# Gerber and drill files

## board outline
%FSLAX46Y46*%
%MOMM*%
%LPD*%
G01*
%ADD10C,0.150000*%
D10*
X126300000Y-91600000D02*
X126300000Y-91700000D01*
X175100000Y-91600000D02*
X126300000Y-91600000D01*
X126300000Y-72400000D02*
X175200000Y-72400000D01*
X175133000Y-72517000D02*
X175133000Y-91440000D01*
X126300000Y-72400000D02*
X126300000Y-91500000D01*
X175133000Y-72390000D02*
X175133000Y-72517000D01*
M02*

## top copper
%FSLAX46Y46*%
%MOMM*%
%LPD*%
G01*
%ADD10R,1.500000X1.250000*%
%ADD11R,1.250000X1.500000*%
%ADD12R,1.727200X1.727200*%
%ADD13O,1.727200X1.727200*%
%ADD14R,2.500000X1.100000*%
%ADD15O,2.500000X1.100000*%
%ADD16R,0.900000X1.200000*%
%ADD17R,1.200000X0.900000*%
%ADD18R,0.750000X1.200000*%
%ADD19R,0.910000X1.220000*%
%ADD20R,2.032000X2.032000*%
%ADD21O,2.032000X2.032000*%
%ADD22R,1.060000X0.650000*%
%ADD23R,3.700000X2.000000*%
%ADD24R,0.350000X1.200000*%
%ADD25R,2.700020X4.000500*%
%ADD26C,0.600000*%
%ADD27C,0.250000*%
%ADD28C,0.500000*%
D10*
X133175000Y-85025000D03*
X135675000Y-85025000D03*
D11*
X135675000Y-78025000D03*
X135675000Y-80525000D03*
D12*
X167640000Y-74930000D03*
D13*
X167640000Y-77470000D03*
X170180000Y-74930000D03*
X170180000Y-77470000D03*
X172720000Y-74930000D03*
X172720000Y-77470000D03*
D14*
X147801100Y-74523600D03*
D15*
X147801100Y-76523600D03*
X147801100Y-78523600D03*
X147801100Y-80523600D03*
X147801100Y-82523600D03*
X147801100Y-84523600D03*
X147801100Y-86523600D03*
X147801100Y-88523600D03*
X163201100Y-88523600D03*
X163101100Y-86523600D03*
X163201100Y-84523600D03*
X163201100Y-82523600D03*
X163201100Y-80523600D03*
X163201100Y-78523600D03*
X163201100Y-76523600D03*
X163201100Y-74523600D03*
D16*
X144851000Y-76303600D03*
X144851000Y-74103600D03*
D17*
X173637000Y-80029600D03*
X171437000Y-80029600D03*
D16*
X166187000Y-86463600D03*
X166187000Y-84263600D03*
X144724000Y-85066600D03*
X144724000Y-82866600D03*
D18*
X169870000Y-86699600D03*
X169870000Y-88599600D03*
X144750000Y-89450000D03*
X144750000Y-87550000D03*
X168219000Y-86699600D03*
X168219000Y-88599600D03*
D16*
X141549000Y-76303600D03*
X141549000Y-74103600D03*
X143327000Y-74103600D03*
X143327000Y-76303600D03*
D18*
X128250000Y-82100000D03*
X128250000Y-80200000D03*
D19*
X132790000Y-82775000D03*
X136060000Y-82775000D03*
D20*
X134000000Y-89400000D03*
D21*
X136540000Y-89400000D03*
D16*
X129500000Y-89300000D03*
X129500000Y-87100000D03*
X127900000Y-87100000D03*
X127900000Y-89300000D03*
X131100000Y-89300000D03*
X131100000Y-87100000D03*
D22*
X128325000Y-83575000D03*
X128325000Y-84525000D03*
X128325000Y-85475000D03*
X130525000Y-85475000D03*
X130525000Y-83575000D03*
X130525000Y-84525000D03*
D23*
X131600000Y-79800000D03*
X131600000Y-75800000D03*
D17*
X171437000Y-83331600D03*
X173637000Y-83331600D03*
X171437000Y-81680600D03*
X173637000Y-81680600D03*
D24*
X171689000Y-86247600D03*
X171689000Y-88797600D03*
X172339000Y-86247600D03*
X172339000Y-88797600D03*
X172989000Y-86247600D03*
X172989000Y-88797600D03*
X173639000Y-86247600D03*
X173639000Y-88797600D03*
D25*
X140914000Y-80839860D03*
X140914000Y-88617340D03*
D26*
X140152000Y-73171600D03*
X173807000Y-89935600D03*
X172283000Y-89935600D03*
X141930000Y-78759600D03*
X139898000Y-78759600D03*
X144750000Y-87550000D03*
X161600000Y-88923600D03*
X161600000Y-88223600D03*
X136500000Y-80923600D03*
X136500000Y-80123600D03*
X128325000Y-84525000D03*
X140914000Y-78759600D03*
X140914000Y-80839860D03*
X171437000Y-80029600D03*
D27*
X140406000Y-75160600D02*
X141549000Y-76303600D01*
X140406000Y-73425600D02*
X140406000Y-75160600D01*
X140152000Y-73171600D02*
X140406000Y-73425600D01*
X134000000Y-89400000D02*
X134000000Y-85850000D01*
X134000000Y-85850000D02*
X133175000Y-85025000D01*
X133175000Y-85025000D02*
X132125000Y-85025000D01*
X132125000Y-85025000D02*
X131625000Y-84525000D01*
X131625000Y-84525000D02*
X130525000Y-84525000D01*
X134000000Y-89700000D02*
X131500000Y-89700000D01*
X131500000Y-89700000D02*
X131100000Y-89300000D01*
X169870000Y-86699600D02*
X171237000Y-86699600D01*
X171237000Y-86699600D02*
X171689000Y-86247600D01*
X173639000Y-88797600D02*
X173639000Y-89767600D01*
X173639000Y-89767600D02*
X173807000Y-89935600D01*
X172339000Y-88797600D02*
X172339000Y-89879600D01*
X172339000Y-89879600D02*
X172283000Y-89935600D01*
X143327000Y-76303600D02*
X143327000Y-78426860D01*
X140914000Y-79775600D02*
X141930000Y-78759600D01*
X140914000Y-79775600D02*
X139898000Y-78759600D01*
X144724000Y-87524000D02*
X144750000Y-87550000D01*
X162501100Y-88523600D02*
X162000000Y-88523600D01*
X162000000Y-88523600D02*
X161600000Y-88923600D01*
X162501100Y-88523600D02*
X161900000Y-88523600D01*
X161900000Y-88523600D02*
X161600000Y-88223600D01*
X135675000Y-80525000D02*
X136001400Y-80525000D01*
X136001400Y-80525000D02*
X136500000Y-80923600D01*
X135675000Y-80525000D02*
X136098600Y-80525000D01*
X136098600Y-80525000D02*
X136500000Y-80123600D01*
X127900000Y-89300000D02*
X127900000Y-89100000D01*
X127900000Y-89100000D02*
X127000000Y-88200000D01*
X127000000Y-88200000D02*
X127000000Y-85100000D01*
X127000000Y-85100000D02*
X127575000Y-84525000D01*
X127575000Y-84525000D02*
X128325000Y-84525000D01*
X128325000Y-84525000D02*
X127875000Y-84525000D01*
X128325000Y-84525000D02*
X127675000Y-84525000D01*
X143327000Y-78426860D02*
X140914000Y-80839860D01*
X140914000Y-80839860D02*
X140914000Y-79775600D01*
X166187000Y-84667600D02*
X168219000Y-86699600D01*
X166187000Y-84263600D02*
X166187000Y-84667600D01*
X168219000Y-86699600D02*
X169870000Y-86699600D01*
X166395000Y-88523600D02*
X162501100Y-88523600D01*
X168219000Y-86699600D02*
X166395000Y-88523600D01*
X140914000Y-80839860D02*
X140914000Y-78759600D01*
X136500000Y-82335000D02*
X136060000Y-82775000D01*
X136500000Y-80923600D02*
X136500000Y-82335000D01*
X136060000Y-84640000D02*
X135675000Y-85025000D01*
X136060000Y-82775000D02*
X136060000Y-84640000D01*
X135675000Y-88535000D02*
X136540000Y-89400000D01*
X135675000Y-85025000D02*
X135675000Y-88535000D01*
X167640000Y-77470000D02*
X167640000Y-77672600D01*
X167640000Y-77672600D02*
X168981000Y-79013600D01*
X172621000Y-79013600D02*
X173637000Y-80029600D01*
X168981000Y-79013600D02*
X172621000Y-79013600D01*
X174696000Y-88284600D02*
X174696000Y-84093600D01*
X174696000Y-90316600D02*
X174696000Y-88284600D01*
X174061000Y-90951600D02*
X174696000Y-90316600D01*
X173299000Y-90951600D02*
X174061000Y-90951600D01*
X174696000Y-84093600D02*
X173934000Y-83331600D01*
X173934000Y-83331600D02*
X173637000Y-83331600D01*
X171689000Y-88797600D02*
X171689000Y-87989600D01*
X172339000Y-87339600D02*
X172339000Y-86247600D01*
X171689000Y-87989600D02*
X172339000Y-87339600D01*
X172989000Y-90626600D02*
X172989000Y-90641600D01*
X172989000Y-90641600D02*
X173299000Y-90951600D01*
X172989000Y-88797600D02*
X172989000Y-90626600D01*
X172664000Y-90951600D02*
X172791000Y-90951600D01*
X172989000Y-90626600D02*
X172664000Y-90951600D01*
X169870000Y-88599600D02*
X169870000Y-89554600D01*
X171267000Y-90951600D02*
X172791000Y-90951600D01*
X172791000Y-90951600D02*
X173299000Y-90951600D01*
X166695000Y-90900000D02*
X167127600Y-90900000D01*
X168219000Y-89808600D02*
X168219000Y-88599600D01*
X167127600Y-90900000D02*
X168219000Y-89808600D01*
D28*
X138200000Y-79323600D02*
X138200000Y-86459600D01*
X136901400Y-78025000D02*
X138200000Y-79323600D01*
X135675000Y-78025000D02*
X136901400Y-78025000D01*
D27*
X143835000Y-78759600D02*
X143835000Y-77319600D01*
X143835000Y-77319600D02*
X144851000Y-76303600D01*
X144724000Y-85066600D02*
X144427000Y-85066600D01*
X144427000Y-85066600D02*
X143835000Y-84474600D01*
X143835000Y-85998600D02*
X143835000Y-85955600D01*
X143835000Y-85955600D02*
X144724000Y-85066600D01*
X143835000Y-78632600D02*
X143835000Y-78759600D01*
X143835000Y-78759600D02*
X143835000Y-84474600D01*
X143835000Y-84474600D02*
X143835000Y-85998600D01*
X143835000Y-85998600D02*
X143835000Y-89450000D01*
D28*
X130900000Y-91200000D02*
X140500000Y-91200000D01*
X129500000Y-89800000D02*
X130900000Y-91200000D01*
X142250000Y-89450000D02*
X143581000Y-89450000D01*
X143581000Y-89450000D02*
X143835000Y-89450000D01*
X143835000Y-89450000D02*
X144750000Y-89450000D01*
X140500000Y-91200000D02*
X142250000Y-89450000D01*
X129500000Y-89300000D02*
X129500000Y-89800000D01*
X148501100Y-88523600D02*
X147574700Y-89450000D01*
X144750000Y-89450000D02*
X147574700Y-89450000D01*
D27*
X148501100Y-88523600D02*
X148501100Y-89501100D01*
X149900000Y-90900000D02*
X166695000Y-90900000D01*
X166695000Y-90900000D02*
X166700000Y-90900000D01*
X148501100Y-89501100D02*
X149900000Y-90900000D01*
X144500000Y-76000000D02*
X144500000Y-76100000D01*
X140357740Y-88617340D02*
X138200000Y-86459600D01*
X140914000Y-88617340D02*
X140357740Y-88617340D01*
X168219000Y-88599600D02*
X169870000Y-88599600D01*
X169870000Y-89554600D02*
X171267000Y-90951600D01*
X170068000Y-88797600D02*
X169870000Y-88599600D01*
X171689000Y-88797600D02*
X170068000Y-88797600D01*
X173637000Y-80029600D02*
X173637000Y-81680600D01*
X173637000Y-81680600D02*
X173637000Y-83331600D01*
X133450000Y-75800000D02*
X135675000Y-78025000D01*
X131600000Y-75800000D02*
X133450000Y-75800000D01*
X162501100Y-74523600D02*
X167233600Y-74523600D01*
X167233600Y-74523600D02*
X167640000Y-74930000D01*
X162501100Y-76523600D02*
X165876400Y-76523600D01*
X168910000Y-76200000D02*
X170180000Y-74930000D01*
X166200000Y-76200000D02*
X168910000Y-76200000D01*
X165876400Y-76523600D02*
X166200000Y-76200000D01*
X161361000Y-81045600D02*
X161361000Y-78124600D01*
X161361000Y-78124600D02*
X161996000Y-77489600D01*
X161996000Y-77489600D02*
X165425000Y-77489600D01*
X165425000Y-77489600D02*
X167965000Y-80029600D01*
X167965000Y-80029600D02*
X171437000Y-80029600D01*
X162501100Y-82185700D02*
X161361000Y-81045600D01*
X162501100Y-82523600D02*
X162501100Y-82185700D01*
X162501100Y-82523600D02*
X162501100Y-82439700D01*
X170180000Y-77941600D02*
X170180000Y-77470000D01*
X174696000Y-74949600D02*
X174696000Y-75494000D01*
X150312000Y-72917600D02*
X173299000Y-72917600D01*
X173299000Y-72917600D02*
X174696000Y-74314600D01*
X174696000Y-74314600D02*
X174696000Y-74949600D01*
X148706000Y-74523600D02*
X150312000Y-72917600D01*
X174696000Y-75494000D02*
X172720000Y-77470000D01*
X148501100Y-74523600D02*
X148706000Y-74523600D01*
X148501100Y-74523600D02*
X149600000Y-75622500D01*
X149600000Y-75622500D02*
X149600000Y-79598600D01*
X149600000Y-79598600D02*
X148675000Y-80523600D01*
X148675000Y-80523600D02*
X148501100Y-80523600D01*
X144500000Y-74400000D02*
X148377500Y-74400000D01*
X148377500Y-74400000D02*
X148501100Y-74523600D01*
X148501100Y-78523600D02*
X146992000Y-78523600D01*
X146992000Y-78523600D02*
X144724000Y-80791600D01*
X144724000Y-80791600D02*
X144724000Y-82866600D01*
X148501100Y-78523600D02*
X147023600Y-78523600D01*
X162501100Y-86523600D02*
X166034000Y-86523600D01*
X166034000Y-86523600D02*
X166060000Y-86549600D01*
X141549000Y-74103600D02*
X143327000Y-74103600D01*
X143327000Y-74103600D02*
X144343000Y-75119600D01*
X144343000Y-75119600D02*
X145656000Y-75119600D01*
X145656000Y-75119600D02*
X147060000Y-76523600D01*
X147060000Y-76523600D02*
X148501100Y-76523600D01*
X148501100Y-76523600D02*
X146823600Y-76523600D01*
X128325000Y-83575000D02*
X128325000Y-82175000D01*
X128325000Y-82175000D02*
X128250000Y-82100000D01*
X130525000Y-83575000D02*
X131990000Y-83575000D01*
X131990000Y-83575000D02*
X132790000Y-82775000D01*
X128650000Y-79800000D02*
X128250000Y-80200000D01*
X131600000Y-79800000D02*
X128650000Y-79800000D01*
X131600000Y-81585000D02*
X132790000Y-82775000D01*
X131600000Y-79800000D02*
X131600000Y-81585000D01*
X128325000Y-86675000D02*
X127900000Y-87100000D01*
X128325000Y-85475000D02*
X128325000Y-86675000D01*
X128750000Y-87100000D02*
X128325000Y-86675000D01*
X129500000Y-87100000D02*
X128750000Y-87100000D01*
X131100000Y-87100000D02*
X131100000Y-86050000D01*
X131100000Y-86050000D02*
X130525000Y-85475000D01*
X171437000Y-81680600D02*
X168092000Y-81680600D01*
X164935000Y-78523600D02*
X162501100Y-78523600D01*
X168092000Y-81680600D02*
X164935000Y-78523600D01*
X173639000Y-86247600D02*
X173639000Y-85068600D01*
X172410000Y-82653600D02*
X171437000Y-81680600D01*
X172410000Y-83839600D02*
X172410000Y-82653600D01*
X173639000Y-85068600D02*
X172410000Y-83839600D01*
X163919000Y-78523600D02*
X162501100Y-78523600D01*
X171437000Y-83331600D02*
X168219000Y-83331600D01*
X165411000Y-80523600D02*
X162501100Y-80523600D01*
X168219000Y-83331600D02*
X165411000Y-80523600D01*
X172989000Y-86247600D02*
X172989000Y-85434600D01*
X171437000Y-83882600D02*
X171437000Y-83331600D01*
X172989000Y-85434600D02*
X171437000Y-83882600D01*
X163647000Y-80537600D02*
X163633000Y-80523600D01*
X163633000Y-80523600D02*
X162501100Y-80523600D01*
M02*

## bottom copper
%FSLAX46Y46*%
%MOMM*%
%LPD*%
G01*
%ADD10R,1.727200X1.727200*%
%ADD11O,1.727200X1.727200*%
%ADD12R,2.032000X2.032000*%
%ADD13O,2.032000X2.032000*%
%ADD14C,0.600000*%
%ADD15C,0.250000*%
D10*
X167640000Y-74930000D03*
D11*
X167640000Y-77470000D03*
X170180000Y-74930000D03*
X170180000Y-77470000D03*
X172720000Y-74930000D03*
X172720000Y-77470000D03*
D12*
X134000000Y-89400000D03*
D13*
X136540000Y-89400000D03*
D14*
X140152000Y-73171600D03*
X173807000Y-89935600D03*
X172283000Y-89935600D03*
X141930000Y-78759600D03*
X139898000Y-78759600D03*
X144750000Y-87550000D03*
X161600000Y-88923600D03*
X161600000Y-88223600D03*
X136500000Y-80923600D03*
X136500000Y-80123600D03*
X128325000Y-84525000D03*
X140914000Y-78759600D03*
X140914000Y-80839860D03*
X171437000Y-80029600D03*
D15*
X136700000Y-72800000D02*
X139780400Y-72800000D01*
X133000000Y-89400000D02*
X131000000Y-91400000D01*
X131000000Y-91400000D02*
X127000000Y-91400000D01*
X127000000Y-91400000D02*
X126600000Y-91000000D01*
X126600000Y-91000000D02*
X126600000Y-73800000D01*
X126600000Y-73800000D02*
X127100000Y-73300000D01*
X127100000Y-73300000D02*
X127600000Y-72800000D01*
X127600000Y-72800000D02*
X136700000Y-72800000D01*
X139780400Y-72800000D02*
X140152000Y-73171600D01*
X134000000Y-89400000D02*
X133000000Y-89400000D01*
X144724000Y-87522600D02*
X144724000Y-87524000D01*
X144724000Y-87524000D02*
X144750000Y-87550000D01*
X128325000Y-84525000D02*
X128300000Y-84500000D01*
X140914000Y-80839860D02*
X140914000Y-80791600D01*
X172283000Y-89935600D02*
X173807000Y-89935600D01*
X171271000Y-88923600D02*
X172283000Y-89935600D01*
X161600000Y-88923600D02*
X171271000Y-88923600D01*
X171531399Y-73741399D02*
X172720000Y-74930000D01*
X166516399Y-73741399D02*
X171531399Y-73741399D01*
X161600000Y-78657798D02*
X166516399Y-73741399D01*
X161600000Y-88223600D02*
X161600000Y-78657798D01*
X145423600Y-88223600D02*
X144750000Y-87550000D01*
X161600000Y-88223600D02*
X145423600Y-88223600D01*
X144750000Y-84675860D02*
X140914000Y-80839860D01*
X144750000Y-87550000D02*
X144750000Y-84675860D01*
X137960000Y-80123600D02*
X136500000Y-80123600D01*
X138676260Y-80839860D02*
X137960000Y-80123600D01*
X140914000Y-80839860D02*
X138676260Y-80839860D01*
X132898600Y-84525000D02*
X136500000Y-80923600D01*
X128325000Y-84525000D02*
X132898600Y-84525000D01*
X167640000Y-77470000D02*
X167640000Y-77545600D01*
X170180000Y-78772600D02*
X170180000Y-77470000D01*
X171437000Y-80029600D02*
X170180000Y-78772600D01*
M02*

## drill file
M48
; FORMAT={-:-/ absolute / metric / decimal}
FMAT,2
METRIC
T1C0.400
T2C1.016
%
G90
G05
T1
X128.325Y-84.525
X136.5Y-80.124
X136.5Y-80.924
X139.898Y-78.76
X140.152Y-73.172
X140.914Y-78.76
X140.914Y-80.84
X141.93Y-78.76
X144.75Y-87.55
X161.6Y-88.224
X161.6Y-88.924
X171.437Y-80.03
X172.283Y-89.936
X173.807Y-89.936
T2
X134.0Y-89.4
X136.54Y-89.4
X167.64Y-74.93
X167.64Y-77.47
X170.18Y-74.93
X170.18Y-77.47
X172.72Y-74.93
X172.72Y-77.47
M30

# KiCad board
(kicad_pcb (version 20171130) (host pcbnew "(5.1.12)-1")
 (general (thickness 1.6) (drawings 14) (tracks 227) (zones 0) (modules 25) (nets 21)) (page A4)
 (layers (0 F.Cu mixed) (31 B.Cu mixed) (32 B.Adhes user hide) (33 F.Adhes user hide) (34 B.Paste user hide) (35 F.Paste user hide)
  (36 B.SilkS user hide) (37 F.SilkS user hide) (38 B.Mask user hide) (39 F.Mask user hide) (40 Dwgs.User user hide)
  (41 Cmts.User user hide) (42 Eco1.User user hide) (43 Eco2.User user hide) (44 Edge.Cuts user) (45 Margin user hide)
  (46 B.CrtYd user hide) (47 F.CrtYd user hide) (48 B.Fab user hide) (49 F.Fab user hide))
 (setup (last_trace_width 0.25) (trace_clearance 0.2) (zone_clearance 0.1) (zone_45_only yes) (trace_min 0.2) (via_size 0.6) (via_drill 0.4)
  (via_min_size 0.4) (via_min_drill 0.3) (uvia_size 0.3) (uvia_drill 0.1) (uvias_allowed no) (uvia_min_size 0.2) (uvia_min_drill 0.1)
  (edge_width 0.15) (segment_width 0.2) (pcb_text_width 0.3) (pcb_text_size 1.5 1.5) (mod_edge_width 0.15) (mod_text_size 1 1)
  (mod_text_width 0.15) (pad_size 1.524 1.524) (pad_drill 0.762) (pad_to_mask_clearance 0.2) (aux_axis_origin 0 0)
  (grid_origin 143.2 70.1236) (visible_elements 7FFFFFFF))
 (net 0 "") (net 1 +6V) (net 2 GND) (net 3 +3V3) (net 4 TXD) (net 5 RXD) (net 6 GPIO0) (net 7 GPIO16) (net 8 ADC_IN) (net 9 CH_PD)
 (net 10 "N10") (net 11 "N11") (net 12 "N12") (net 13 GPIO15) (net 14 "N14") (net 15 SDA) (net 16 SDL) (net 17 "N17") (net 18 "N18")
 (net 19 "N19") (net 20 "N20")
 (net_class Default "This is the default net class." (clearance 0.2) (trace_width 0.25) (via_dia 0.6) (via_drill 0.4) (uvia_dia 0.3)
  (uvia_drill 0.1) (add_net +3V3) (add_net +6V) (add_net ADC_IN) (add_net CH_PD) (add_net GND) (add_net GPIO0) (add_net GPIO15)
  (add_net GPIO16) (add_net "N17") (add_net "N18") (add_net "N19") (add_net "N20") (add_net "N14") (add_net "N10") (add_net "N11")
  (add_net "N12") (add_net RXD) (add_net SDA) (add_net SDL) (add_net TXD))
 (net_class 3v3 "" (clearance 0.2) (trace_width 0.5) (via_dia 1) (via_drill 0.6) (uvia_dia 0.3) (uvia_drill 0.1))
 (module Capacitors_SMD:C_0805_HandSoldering (layer F.Cu) (at 134.425 85.025)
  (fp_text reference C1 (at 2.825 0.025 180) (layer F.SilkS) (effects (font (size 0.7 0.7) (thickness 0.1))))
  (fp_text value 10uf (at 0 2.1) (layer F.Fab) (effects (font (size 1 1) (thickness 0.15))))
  (pad 1 smd rect (at -1.25 0) (size 1.5 1.25) (layers F.Cu F.Paste F.Mask) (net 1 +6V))
  (pad 2 smd rect (at 1.25 0) (size 1.5 1.25) (layers F.Cu F.Paste F.Mask) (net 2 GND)))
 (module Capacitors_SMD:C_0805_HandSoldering (layer F.Cu) (at 135.675 79.275 270)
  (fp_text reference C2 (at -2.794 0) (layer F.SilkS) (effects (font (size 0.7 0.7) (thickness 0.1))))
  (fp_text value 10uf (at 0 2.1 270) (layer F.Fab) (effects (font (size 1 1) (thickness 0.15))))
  (pad 1 smd rect (at -1.25 0 270) (size 1.5 1.25) (layers F.Cu F.Paste F.Mask) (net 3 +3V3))
  (pad 2 smd rect (at 1.25 0 270) (size 1.5 1.25) (layers F.Cu F.Paste F.Mask) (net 2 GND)))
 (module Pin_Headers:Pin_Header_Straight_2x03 (layer B.Cu) (at 167.64 74.93 270)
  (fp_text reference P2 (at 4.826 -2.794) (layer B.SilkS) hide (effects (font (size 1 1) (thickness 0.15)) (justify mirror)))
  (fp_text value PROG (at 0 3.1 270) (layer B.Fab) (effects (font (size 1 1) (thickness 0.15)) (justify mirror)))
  (pad 1 thru_hole rect (at 0 0 270) (size 1.7272 1.7272) (drill 1.016) (layers *.Cu *.Mask B.SilkS) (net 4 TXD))
  (pad 2 thru_hole oval (at 2.54 0 270) (size 1.7272 1.7272) (drill 1.016) (layers *.Cu *.Mask B.SilkS) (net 3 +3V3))
  (pad 3 thru_hole oval (at 0 -2.54 270) (size 1.7272 1.7272) (drill 1.016) (layers *.Cu *.Mask B.SilkS) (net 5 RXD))
  (pad 4 thru_hole oval (at 2.54 -2.54 270) (size 1.7272 1.7272) (drill 1.016) (layers *.Cu *.Mask B.SilkS) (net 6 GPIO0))
  (pad 5 thru_hole oval (at 0 -5.08 270) (size 1.7272 1.7272) (drill 1.016) (layers *.Cu *.Mask B.SilkS) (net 2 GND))
  (pad 6 thru_hole oval (at 2.54 -5.08 270) (size 1.7272 1.7272) (drill 1.016) (layers *.Cu *.Mask B.SilkS) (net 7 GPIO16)))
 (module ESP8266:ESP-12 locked (layer F.Cu) (at 148.5011 74.5236)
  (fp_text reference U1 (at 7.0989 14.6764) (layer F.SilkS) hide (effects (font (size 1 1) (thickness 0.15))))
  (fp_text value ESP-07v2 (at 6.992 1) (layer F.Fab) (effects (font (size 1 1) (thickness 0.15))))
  (pad 1 smd rect (at 0 0) (size 2.5 1.1) (drill (offset -0.7 0)) (layers F.Cu F.Paste F.Mask) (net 7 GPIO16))
  (pad 2 smd oval (at 0 2) (size 2.5 1.1) (drill (offset -0.7 0)) (layers F.Cu F.Paste F.Mask) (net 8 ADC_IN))
  (pad 3 smd oval (at 0 4) (size 2.5 1.1) (drill (offset -0.7 0)) (layers F.Cu F.Paste F.Mask) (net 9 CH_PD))
  (pad 4 smd oval (at 0 6) (size 2.5 1.1) (drill (offset -0.7 0)) (layers F.Cu F.Paste F.Mask) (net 7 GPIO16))
  (pad 5 smd oval (at 0 8) (size 2.5 1.1) (drill (offset -0.7 0)) (layers F.Cu F.Paste F.Mask) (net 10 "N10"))
  (pad 6 smd oval (at 0 10) (size 2.5 1.1) (drill (offset -0.7 0)) (layers F.Cu F.Paste F.Mask) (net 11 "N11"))
  (pad 7 smd oval (at 0 12) (size 2.5 1.1) (drill (offset -0.7 0)) (layers F.Cu F.Paste F.Mask) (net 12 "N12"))
  (pad 8 smd oval (at 0 14) (size 2.5 1.1) (drill (offset -0.7 0)) (layers F.Cu F.Paste F.Mask) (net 3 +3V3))
  (pad 9 smd oval (at 14 14) (size 2.5 1.1) (drill (offset 0.7 0)) (layers F.Cu F.Paste F.Mask) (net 2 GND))
  (pad 10 smd oval (at 14 12) (size 2.5 1.1) (drill (offset 0.6 0)) (layers F.Cu F.Paste F.Mask) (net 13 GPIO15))
  (pad 11 smd oval (at 14 10) (size 2.5 1.1) (drill (offset 0.7 0)) (layers F.Cu F.Paste F.Mask) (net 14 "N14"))
  (pad 12 smd oval (at 14 8) (size 2.5 1.1) (drill (offset 0.7 0)) (layers F.Cu F.Paste F.Mask) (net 6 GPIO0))
  (pad 13 smd oval (at 14 6) (size 2.5 1.1) (drill (offset 0.7 0)) (layers F.Cu F.Paste F.Mask) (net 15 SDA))
  (pad 14 smd oval (at 14 4) (size 2.5 1.1) (drill (offset 0.7 0)) (layers F.Cu F.Paste F.Mask) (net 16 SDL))
  (pad 15 smd oval (at 14 2) (size 2.5 1.1) (drill (offset 0.7 0)) (layers F.Cu F.Paste F.Mask) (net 5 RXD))
  (pad 16 smd oval (at 14 0) (size 2.5 1.1) (drill (offset 0.7 0)) (layers F.Cu F.Paste F.Mask) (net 4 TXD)))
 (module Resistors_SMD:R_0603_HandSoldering (layer F.Cu) (at 144.851 75.2036 90)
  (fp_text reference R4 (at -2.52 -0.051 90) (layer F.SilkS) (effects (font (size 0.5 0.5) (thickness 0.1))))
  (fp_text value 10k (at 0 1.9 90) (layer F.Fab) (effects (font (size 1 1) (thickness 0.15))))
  (pad 1 smd rect (at -1.1 0 90) (size 1.2 0.9) (layers F.Cu F.Paste F.Mask) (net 3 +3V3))
  (pad 2 smd rect (at 1.1 0 90) (size 1.2 0.9) (layers F.Cu F.Paste F.Mask) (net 7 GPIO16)))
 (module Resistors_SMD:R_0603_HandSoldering (layer F.Cu) (at 172.537 80.0296 180)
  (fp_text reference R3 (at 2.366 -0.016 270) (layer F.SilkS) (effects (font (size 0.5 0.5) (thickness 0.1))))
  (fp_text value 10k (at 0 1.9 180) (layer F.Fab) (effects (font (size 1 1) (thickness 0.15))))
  (pad 1 smd rect (at -1.1 0 180) (size 1.2 0.9) (layers F.Cu F.Paste F.Mask) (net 3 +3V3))
  (pad 2 smd rect (at 1.1 0 180) (size 1.2 0.9) (layers F.Cu F.Paste F.Mask) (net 6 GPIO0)))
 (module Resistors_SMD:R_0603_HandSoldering (layer F.Cu) (at 166.187 85.3636 90)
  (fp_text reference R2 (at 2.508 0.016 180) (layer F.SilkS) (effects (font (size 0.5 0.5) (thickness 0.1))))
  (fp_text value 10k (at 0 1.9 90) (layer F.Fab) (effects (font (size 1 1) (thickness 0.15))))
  (pad 1 smd rect (at -1.1 0 90) (size 1.2 0.9) (layers F.Cu F.Paste F.Mask) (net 13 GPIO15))
  (pad 2 smd rect (at 1.1 0 90) (size 1.2 0.9) (layers F.Cu F.Paste F.Mask) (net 2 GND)))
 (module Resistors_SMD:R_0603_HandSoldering (layer F.Cu) (at 144.724 83.9666 90)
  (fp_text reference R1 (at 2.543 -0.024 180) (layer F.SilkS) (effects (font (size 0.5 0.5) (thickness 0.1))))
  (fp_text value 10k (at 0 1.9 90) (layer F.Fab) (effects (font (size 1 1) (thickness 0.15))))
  (pad 1 smd rect (at -1.1 0 90) (size 1.2 0.9) (layers F.Cu F.Paste F.Mask) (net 3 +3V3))
  (pad 2 smd rect (at 1.1 0 90) (size 1.2 0.9) (layers F.Cu F.Paste F.Mask) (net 9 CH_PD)))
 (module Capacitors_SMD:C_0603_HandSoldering (layer F.Cu) (at 169.87 87.6496 270)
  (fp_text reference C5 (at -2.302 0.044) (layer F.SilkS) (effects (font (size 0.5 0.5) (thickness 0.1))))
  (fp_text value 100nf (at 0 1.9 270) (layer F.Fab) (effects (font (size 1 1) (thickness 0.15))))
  (pad 1 smd rect (at -0.95 0 270) (size 1.2 0.75) (layers F.Cu F.Paste F.Mask) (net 2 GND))
  (pad 2 smd rect (at 0.95 0 270) (size 1.2 0.75) (layers F.Cu F.Paste F.Mask) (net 3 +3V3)))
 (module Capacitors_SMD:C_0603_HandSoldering (layer F.Cu) (at 144.75 88.5 90)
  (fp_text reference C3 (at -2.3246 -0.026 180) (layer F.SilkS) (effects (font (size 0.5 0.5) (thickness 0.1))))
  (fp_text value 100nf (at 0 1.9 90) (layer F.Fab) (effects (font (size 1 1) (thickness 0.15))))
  (pad 1 smd rect (at -0.95 0 90) (size 1.2 0.75) (layers F.Cu F.Paste F.Mask) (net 3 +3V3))
  (pad 2 smd rect (at 0.95 0 90) (size 1.2 0.75) (layers F.Cu F.Paste F.Mask) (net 2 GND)))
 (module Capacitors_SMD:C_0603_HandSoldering (layer F.Cu) (at 168.219 87.6496 270)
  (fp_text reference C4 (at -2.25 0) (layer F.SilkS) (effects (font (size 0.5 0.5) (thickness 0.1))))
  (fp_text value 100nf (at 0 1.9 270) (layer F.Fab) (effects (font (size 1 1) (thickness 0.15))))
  (pad 1 smd rect (at -0.95 0 270) (size 1.2 0.75) (layers F.Cu F.Paste F.Mask) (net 2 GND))
  (pad 2 smd rect (at 0.95 0 270) (size 1.2 0.75) (layers F.Cu F.Paste F.Mask) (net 3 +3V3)))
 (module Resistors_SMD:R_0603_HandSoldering (layer F.Cu) (at 141.549 75.2036 90)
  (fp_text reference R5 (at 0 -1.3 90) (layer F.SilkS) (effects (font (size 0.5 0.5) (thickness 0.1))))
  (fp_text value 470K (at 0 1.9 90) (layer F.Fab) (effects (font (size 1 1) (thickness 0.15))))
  (pad 1 smd rect (at -1.1 0 90) (size 1.2 0.9) (layers F.Cu F.Paste F.Mask) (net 1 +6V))
  (pad 2 smd rect (at 1.1 0 90) (size 1.2 0.9) (layers F.Cu F.Paste F.Mask) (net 8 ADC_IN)))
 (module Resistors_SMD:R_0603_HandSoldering (layer F.Cu) (at 143.327 75.2036 270)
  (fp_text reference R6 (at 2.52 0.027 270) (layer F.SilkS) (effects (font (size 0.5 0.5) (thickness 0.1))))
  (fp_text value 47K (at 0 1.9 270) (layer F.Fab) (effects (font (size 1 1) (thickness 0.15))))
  (pad 1 smd rect (at -1.1 0 270) (size 1.2 0.9) (layers F.Cu F.Paste F.Mask) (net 8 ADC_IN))
  (pad 2 smd rect (at 1.1 0 270) (size 1.2 0.9) (layers F.Cu F.Paste F.Mask) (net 2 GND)))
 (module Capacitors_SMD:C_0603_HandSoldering (layer F.Cu) (at 128.25 81.15 90)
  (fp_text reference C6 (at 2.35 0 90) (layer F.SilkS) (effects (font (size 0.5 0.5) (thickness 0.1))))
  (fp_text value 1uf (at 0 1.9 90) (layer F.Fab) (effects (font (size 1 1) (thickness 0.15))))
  (pad 1 smd rect (at -0.95 0 90) (size 1.2 0.75) (layers F.Cu F.Paste F.Mask) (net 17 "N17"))
  (pad 2 smd rect (at 0.95 0 90) (size 1.2 0.75) (layers F.Cu F.Paste F.Mask) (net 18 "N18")))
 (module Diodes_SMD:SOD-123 (layer F.Cu) (at 134.425 82.775)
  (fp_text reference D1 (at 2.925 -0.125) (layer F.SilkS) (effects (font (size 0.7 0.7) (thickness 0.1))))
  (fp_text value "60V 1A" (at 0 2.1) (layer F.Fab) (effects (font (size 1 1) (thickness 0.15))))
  (pad 1 smd rect (at -1.635 0) (size 0.91 1.22) (layers F.Cu F.Paste F.Mask) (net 18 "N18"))
  (pad 2 smd rect (at 1.635 0) (size 0.91 1.22) (layers F.Cu F.Paste F.Mask) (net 2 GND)))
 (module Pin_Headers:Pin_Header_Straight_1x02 (layer F.Cu) (at 134 89.4 90)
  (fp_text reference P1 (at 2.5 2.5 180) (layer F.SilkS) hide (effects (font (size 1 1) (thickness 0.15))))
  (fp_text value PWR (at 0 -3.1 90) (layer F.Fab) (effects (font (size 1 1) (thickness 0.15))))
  (pad 1 thru_hole rect (at 0 0 90) (size 2.032 2.032) (drill 1.016) (layers *.Cu *.Mask F.SilkS) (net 1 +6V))
  (pad 2 thru_hole oval (at 0 2.54 90) (size 2.032 2.032) (drill 1.016) (layers *.Cu *.Mask F.SilkS) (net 2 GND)))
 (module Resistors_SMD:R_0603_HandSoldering (layer F.Cu) (at 129.5 88.2 90)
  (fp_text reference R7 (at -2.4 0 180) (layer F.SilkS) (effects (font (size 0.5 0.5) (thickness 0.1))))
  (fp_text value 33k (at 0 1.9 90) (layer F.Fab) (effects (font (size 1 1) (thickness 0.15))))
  (pad 1 smd rect (at -1.1 0 90) (size 1.2 0.9) (layers F.Cu F.Paste F.Mask) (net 3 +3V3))
  (pad 2 smd rect (at 1.1 0 90) (size 1.2 0.9) (layers F.Cu F.Paste F.Mask) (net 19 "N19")))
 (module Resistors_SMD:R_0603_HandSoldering (layer F.Cu) (at 127.9 88.2 270)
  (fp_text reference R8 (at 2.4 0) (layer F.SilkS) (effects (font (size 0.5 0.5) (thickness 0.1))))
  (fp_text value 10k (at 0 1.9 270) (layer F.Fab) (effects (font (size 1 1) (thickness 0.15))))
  (pad 1 smd rect (at -1.1 0 270) (size 1.2 0.9) (layers F.Cu F.Paste F.Mask) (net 19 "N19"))
  (pad 2 smd rect (at 1.1 0 270) (size 1.2 0.9) (layers F.Cu F.Paste F.Mask) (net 2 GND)))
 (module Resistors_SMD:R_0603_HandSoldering (layer F.Cu) (at 131.1 88.2 90)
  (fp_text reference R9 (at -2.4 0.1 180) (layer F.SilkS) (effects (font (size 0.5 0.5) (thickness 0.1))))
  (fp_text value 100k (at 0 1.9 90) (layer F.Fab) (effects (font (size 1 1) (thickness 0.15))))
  (pad 1 smd rect (at -1.1 0 90) (size 1.2 0.9) (layers F.Cu F.Paste F.Mask) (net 1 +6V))
  (pad 2 smd rect (at 1.1 0 90) (size 1.2 0.9) (layers F.Cu F.Paste F.Mask) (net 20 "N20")))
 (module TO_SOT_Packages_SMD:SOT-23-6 (layer F.Cu) (at 129.425 84.525) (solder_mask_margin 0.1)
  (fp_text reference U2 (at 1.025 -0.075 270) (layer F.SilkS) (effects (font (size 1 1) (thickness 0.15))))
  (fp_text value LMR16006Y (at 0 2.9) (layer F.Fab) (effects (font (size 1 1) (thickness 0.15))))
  (pad 1 smd rect (at -1.1 -0.95) (size 1.06 0.65) (layers F.Cu F.Paste F.Mask) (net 17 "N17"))
  (pad 2 smd rect (at -1.1 0) (size 1.06 0.65) (layers F.Cu F.Paste F.Mask) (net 2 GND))
  (pad 3 smd rect (at -1.1 0.95) (size 1.06 0.65) (layers F.Cu F.Paste F.Mask) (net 19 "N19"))
  (pad 4 smd rect (at 1.1 0.95) (size 1.06 0.65) (layers F.Cu F.Paste F.Mask) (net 20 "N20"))
  (pad 6 smd rect (at 1.1 -0.95) (size 1.06 0.65) (layers F.Cu F.Paste F.Mask) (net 18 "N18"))
  (pad 5 smd rect (at 1.1 0) (size 1.06 0.65) (layers F.Cu F.Paste F.Mask) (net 1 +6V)))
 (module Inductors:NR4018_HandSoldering (layer F.Cu) (at 131.6 77.8 90)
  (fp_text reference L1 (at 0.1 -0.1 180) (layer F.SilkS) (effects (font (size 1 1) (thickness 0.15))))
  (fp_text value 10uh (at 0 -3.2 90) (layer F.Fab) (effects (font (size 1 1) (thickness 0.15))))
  (pad 1 smd rect (at -2 0 90) (size 2 3.7) (layers F.Cu F.Paste F.Mask) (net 18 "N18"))
  (pad 2 smd rect (at 2 0 90) (size 2 3.7) (layers F.Cu F.Paste F.Mask) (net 3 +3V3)))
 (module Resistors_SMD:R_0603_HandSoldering (layer F.Cu) (at 172.537 83.3316)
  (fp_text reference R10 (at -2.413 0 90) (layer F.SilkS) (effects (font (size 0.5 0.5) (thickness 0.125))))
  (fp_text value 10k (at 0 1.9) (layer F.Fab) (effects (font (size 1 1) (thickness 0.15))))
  (pad 1 smd rect (at -1.1 0) (size 1.2 0.9) (layers F.Cu F.Paste F.Mask) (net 15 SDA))
  (pad 2 smd rect (at 1.1 0) (size 1.2 0.9) (layers F.Cu F.Paste F.Mask) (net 3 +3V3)))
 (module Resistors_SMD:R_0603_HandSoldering (layer F.Cu) (at 172.537 81.6806)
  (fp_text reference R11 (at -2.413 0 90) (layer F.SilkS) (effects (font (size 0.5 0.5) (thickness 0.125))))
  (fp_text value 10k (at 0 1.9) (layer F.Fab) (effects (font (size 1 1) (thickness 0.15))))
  (pad 1 smd rect (at -1.1 0) (size 1.2 0.9) (layers F.Cu F.Paste F.Mask) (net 16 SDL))
  (pad 2 smd rect (at 1.1 0) (size 1.2 0.9) (layers F.Cu F.Paste F.Mask) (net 3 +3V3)))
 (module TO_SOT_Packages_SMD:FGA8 (layer F.Cu) (at 172.664 87.5226)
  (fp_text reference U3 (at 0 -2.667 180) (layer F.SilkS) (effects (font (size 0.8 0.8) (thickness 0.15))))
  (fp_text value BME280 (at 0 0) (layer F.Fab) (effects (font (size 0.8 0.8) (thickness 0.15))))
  (pad 1 smd rect (at -0.975 -1.275) (size 0.35 1.2) (layers F.Cu F.Paste F.Mask) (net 2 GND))
  (pad 8 smd rect (at -0.975 1.275) (size 0.35 1.2) (layers F.Cu F.Paste F.Mask) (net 3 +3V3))
  (pad 2 smd rect (at -0.325 -1.275) (size 0.35 1.2) (layers F.Cu F.Paste F.Mask) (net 3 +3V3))
  (pad 7 smd rect (at -0.325 1.275) (size 0.35 1.2) (layers F.Cu F.Paste F.Mask) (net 2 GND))
  (pad 3 smd rect (at 0.325 -1.275) (size 0.35 1.2) (layers F.Cu F.Paste F.Mask) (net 15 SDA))
  (pad 6 smd rect (at 0.325 1.275) (size 0.35 1.2) (layers F.Cu F.Paste F.Mask) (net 3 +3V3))
  (pad 4 smd rect (at 0.975 -1.275) (size 0.35 1.2) (layers F.Cu F.Paste F.Mask) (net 16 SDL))
  (pad 5 smd rect (at 0.975 1.275) (size 0.35 1.2) (layers F.Cu F.Paste F.Mask) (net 2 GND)))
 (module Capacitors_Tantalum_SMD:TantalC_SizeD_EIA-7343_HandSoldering (layer F.Cu) (at 140.914 84.7286 90)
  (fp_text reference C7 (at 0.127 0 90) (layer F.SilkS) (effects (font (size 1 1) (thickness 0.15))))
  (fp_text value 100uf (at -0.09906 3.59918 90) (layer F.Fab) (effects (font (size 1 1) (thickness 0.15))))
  (pad 2 smd rect (at 3.88874 0 90) (size 4.0005 2.70002) (layers F.Cu F.Paste F.Mask) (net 2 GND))
  (pad 1 smd rect (at -3.88874 0 90) (size 4.0005 2.70002) (layers F.Cu F.Paste F.Mask) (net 3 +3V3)))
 (gr_line (start 126.3 91.6) (end 126.3 91.7) (angle 90) (layer Edge.Cuts) (width 0.15))
 (gr_line (start 175.1 91.6) (end 126.3 91.6) (angle 90) (layer Edge.Cuts) (width 0.15))
 (gr_line (start 126.3 72.4) (end 175.2 72.4) (angle 90) (layer Edge.Cuts) (width 0.15))
 (gr_line (start 175.133 72.517) (end 175.133 91.44) (angle 90) (layer Edge.Cuts) (width 0.15))
 (gr_line (start 126.3 72.4) (end 126.3 91.5) (angle 90) (layer Edge.Cuts) (width 0.15))
 (gr_line (start 175.133 72.39) (end 175.133 72.517) (angle 90) (layer Edge.Cuts) (width 0.15))
 (segment (start 136.7 72.8) (end 139.7804 72.8) (width 0.25) (layer B.Cu) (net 1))
 (segment (start 133 89.4) (end 131 91.4) (width 0.25) (layer B.Cu) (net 1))
 (segment (start 131 91.4) (end 127 91.4) (width 0.25) (layer B.Cu) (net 1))
 (segment (start 127 91.4) (end 126.6 91) (width 0.25) (layer B.Cu) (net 1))
 (segment (start 126.6 91) (end 126.6 73.8) (width 0.25) (layer B.Cu) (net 1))
 (segment (start 126.6 73.8) (end 127.1 73.3) (width 0.25) (layer B.Cu) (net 1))
 (segment (start 127.1 73.3) (end 127.6 72.8) (width 0.25) (layer B.Cu) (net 1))
 (segment (start 127.6 72.8) (end 136.7 72.8) (width 0.25) (layer B.Cu) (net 1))
 (segment (start 140.406 75.1606) (end 141.549 76.3036) (width 0.25) (layer F.Cu) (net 1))
 (segment (start 140.406 73.4256) (end 140.406 75.1606) (width 0.25) (layer F.Cu) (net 1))
 (segment (start 140.152 73.1716) (end 140.406 73.4256) (width 0.25) (layer F.Cu) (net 1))
 (segment (start 139.7804 72.8) (end 140.152 73.1716) (width 0.25) (layer B.Cu) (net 1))
 (segment (start 134 89.4) (end 134 85.85) (width 0.25) (layer F.Cu) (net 1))
 (segment (start 134 85.85) (end 133.175 85.025) (width 0.25) (layer F.Cu) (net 1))
 (segment (start 134 89.4) (end 133 89.4) (width 0.25) (layer B.Cu) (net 1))
 (segment (start 133.175 85.025) (end 132.125 85.025) (width 0.25) (layer F.Cu) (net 1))
 (segment (start 132.125 85.025) (end 131.625 84.525) (width 0.25) (layer F.Cu) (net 1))
 (segment (start 131.625 84.525) (end 130.525 84.525) (width 0.25) (layer F.Cu) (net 1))
 (segment (start 134 89.7) (end 131.5 89.7) (width 0.25) (layer F.Cu) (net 1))
 (segment (start 131.5 89.7) (end 131.1 89.3) (width 0.25) (layer F.Cu) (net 1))
 (segment (start 169.87 86.6996) (end 171.237 86.6996) (width 0.25) (layer F.Cu) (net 2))
 (segment (start 171.237 86.6996) (end 171.689 86.2476) (width 0.25) (layer F.Cu) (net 2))
 (segment (start 173.639 88.7976) (end 173.639 89.7676) (width 0.25) (layer F.Cu) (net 2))
 (segment (start 173.639 89.7676) (end 173.807 89.9356) (width 0.25) (layer F.Cu) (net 2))
 (segment (start 172.339 88.7976) (end 172.339 89.8796) (width 0.25) (layer F.Cu) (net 2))
 (segment (start 172.339 89.8796) (end 172.283 89.9356) (width 0.25) (layer F.Cu) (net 2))
 (segment (start 143.327 76.3036) (end 143.327 78.42686) (width 0.25) (layer F.Cu) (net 2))
 (segment (start 140.914 79.7756) (end 141.93 78.7596) (width 0.25) (layer F.Cu) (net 2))
 (segment (start 140.914 79.7756) (end 139.898 78.7596) (width 0.25) (layer F.Cu) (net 2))
 (segment (start 144.724 87.524) (end 144.75 87.55) (width 0.25) (layer F.Cu) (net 2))
 (segment (start 144.724 87.5226) (end 144.724 87.524) (width 0.25) (layer B.Cu) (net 2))
 (segment (start 144.724 87.524) (end 144.75 87.55) (width 0.25) (layer B.Cu) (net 2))
 (segment (start 162.5011 88.5236) (end 162 88.5236) (width 0.25) (layer F.Cu) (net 2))
 (segment (start 162 88.5236) (end 161.6 88.9236) (width 0.25) (layer F.Cu) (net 2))
 (segment (start 162.5011 88.5236) (end 161.9 88.5236) (width 0.25) (layer F.Cu) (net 2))
 (segment (start 161.9 88.5236) (end 161.6 88.2236) (width 0.25) (layer F.Cu) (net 2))
 (segment (start 135.675 80.525) (end 136.0014 80.525) (width 0.25) (layer F.Cu) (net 2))
 (segment (start 136.0014 80.525) (end 136.5 80.9236) (width 0.25) (layer F.Cu) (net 2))
 (segment (start 135.675 80.525) (end 136.0986 80.525) (width 0.25) (layer F.Cu) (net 2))
 (segment (start 136.0986 80.525) (end 136.5 80.1236) (width 0.25) (layer F.Cu) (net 2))
 (segment (start 128.325 84.525) (end 128.3 84.5) (width 0.25) (layer B.Cu) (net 2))
 (segment (start 127.9 89.3) (end 127.9 89.1) (width 0.25) (layer F.Cu) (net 2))
 (segment (start 127.9 89.1) (end 127 88.2) (width 0.25) (layer F.Cu) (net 2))
 (segment (start 127 88.2) (end 127 85.1) (width 0.25) (layer F.Cu) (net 2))
 (segment (start 127 85.1) (end 127.575 84.525) (width 0.25) (layer F.Cu) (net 2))
 (segment (start 127.575 84.525) (end 128.325 84.525) (width 0.25) (layer F.Cu) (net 2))
 (segment (start 128.325 84.525) (end 127.875 84.525) (width 0.25) (layer F.Cu) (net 2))
 (segment (start 128.325 84.525) (end 127.675 84.525) (width 0.25) (layer F.Cu) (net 2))
 (segment (start 143.327 78.42686) (end 140.914 80.83986) (width 0.25) (layer F.Cu) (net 2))
 (segment (start 140.914 80.83986) (end 140.914 79.7756) (width 0.25) (layer F.Cu) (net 2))
 (segment (start 140.914 80.83986) (end 140.914 80.7916) (width 0.25) (layer B.Cu) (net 2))
 (segment (start 166.187 84.6676) (end 168.219 86.6996) (width 0.25) (layer F.Cu) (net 2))
 (segment (start 166.187 84.2636) (end 166.187 84.6676) (width 0.25) (layer F.Cu) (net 2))
 (segment (start 168.219 86.6996) (end 169.87 86.6996) (width 0.25) (layer F.Cu) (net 2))
 (segment (start 172.283 89.9356) (end 173.807 89.9356) (width 0.25) (layer B.Cu) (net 2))
 (segment (start 171.271 88.9236) (end 172.283 89.9356) (width 0.25) (layer B.Cu) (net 2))
 (segment (start 161.6 88.9236) (end 171.271 88.9236) (width 0.25) (layer B.Cu) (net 2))
 (segment (start 171.531399 73.741399) (end 172.72 74.93) (width 0.25) (layer B.Cu) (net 2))
 (segment (start 166.516399 73.741399) (end 171.531399 73.741399) (width 0.25) (layer B.Cu) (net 2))
 (segment (start 161.6 78.657798) (end 166.516399 73.741399) (width 0.25) (layer B.Cu) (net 2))
 (segment (start 161.6 88.2236) (end 161.6 78.657798) (width 0.25) (layer B.Cu) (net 2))
 (segment (start 166.395 88.5236) (end 162.5011 88.5236) (width 0.25) (layer F.Cu) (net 2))
 (segment (start 168.219 86.6996) (end 166.395 88.5236) (width 0.25) (layer F.Cu) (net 2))
 (segment (start 145.4236 88.2236) (end 144.75 87.55) (width 0.25) (layer B.Cu) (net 2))
 (segment (start 161.6 88.2236) (end 145.4236 88.2236) (width 0.25) (layer B.Cu) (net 2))
 (segment (start 140.914 80.83986) (end 140.914 78.7596) (width 0.25) (layer F.Cu) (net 2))
 (segment (start 144.75 84.67586) (end 140.914 80.83986) (width 0.25) (layer B.Cu) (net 2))
 (segment (start 144.75 87.55) (end 144.75 84.67586) (width 0.25) (layer B.Cu) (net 2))
 (segment (start 137.96 80.1236) (end 136.5 80.1236) (width 0.25) (layer B.Cu) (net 2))
 (segment (start 138.67626 80.83986) (end 137.96 80.1236) (width 0.25) (layer B.Cu) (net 2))
 (segment (start 140.914 80.83986) (end 138.67626 80.83986) (width 0.25) (layer B.Cu) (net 2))
 (segment (start 136.5 82.335) (end 136.06 82.775) (width 0.25) (layer F.Cu) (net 2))
 (segment (start 136.5 80.9236) (end 136.5 82.335) (width 0.25) (layer F.Cu) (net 2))
 (segment (start 136.06 84.64) (end 135.675 85.025) (width 0.25) (layer F.Cu) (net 2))
 (segment (start 136.06 82.775) (end 136.06 84.64) (width 0.25) (layer F.Cu) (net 2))
 (segment (start 132.8986 84.525) (end 136.5 80.9236) (width 0.25) (layer B.Cu) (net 2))
 (segment (start 128.325 84.525) (end 132.8986 84.525) (width 0.25) (layer B.Cu) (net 2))
 (segment (start 135.675 88.535) (end 136.54 89.4) (width 0.25) (layer F.Cu) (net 2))
 (segment (start 135.675 85.025) (end 135.675 88.535) (width 0.25) (layer F.Cu) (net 2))
 (segment (start 167.64 77.47) (end 167.64 77.6726) (width 0.25) (layer F.Cu) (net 3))
 (segment (start 167.64 77.6726) (end 168.981 79.0136) (width 0.25) (layer F.Cu) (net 3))
 (segment (start 172.621 79.0136) (end 173.637 80.0296) (width 0.25) (layer F.Cu) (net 3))
 (segment (start 168.981 79.0136) (end 172.621 79.0136) (width 0.25) (layer F.Cu) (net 3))
 (segment (start 167.64 77.47) (end 167.64 77.5456) (width 0.25) (layer B.Cu) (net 3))
 (segment (start 174.696 88.2846) (end 174.696 84.0936) (width 0.25) (layer F.Cu) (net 3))
 (segment (start 174.696 90.3166) (end 174.696 88.2846) (width 0.25) (layer F.Cu) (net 3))
 (segment (start 174.061 90.9516) (end 174.696 90.3166) (width 0.25) (layer F.Cu) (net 3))
 (segment (start 173.299 90.9516) (end 174.061 90.9516) (width 0.25) (layer F.Cu) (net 3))
 (segment (start 174.696 84.0936) (end 173.934 83.3316) (width 0.25) (layer F.Cu) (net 3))
 (segment (start 173.934 83.3316) (end 173.637 83.3316) (width 0.25) (layer F.Cu) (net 3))
 (segment (start 171.689 88.7976) (end 171.689 87.9896) (width 0.25) (layer F.Cu) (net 3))
 (segment (start 172.339 87.3396) (end 172.339 86.2476) (width 0.25) (layer F.Cu) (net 3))
 (segment (start 171.689 87.9896) (end 172.339 87.3396) (width 0.25) (layer F.Cu) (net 3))
 (segment (start 172.989 90.6266) (end 172.989 90.6416) (width 0.25) (layer F.Cu) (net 3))
 (segment (start 172.989 90.6416) (end 173.299 90.9516) (width 0.25) (layer F.Cu) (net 3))
 (segment (start 172.989 88.7976) (end 172.989 90.6266) (width 0.25) (layer F.Cu) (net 3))
 (segment (start 172.664 90.9516) (end 172.791 90.9516) (width 0.25) (layer F.Cu) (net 3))
 (segment (start 172.989 90.6266) (end 172.664 90.9516) (width 0.25) (layer F.Cu) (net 3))
 (segment (start 169.87 88.5996) (end 169.87 89.5546) (width 0.25) (layer F.Cu) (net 3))
 (segment (start 171.267 90.9516) (end 172.791 90.9516) (width 0.25) (layer F.Cu) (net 3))
 (segment (start 172.791 90.9516) (end 173.299 90.9516) (width 0.25) (layer F.Cu) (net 3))
 (segment (start 166.695 90.9) (end 167.1276 90.9) (width 0.25) (layer F.Cu) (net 3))
 (segment (start 168.219 89.8086) (end 168.219 88.5996) (width 0.25) (layer F.Cu) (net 3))
 (segment (start 167.1276 90.9) (end 168.219 89.8086) (width 0.25) (layer F.Cu) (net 3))
 (segment (start 138.2 79.3236) (end 138.2 86.4596) (width 0.5) (layer F.Cu) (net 3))
 (segment (start 136.9014 78.025) (end 138.2 79.3236) (width 0.5) (layer F.Cu) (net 3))
 (segment (start 135.675 78.025) (end 136.9014 78.025) (width 0.5) (layer F.Cu) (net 3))
 (segment (start 143.835 78.7596) (end 143.835 77.3196) (width 0.25) (layer F.Cu) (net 3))
 (segment (start 143.835 77.3196) (end 144.851 76.3036) (width 0.25) (layer F.Cu) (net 3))
 (segment (start 144.724 85.0666) (end 144.427 85.0666) (width 0.25) (layer F.Cu) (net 3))
 (segment (start 144.427 85.0666) (end 143.835 84.4746) (width 0.25) (layer F.Cu) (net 3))
 (segment (start 143.835 85.9986) (end 143.835 85.9556) (width 0.25) (layer F.Cu) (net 3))
 (segment (start 143.835 85.9556) (end 144.724 85.0666) (width 0.25) (layer F.Cu) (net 3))
 (segment (start 143.835 78.6326) (end 143.835 78.7596) (width 0.25) (layer F.Cu) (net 3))
 (segment (start 143.835 78.7596) (end 143.835 84.4746) (width 0.25) (layer F.Cu) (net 3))
 (segment (start 143.835 84.4746) (end 143.835 85.9986) (width 0.25) (layer F.Cu) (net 3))
 (segment (start 143.835 85.9986) (end 143.835 89.45) (width 0.25) (layer F.Cu) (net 3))
 (segment (start 130.9 91.2) (end 140.5 91.2) (width 0.5) (layer F.Cu) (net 3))
 (segment (start 129.5 89.8) (end 130.9 91.2) (width 0.5) (layer F.Cu) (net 3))
 (segment (start 142.25 89.45) (end 143.581 89.45) (width 0.5) (layer F.Cu) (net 3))
 (segment (start 143.581 89.45) (end 143.835 89.45) (width 0.5) (layer F.Cu) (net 3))
 (segment (start 143.835 89.45) (end 144.75 89.45) (width 0.5) (layer F.Cu) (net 3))
 (segment (start 140.5 91.2) (end 142.25 89.45) (width 0.5) (layer F.Cu) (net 3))
 (segment (start 129.5 89.3) (end 129.5 89.8) (width 0.5) (layer F.Cu) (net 3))
 (segment (start 148.5011 88.5236) (end 147.5747 89.45) (width 0.5) (layer F.Cu) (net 3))
 (segment (start 144.75 89.45) (end 147.5747 89.45) (width 0.5) (layer F.Cu) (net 3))
 (segment (start 148.5011 88.5236) (end 148.5011 89.5011) (width 0.25) (layer F.Cu) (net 3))
 (segment (start 149.9 90.9) (end 166.695 90.9) (width 0.25) (layer F.Cu) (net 3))
 (segment (start 166.695 90.9) (end 166.7 90.9) (width 0.25) (layer F.Cu) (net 3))
 (segment (start 148.5011 89.5011) (end 149.9 90.9) (width 0.25) (layer F.Cu) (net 3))
 (segment (start 144.5 76) (end 144.5 76.1) (width 0.25) (layer F.Cu) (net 3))
 (segment (start 140.35774 88.61734) (end 138.2 86.4596) (width 0.25) (layer F.Cu) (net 3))
 (segment (start 140.914 88.61734) (end 140.35774 88.61734) (width 0.25) (layer F.Cu) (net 3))
 (segment (start 168.219 88.5996) (end 169.87 88.5996) (width 0.25) (layer F.Cu) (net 3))
 (segment (start 169.87 89.5546) (end 171.267 90.9516) (width 0.25) (layer F.Cu) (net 3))
 (segment (start 170.068 88.7976) (end 169.87 88.5996) (width 0.25) (layer F.Cu) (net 3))
 (segment (start 171.689 88.7976) (end 170.068 88.7976) (width 0.25) (layer F.Cu) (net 3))
 (segment (start 173.637 80.0296) (end 173.637 81.6806) (width 0.25) (layer F.Cu) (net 3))
 (segment (start 173.637 81.6806) (end 173.637 83.3316) (width 0.25) (layer F.Cu) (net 3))
 (segment (start 133.45 75.8) (end 135.675 78.025) (width 0.25) (layer F.Cu) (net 3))
 (segment (start 131.6 75.8) (end 133.45 75.8) (width 0.25) (layer F.Cu) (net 3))
 (segment (start 162.5011 74.5236) (end 167.2336 74.5236) (width 0.25) (layer F.Cu) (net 4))
 (segment (start 167.2336 74.5236) (end 167.64 74.93) (width 0.25) (layer F.Cu) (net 4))
 (segment (start 162.5011 76.5236) (end 165.8764 76.5236) (width 0.25) (layer F.Cu) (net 5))
 (segment (start 168.91 76.2) (end 170.18 74.93) (width 0.25) (layer F.Cu) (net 5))
 (segment (start 166.2 76.2) (end 168.91 76.2) (width 0.25) (layer F.Cu) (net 5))
 (segment (start 165.8764 76.5236) (end 166.2 76.2) (width 0.25) (layer F.Cu) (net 5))
 (segment (start 161.361 81.0456) (end 161.361 78.1246) (width 0.25) (layer F.Cu) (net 6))
 (segment (start 161.361 78.1246) (end 161.996 77.4896) (width 0.25) (layer F.Cu) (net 6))
 (segment (start 161.996 77.4896) (end 165.425 77.4896) (width 0.25) (layer F.Cu) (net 6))
 (segment (start 165.425 77.4896) (end 167.965 80.0296) (width 0.25) (layer F.Cu) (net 6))
 (segment (start 167.965 80.0296) (end 171.437 80.0296) (width 0.25) (layer F.Cu) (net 6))
 (segment (start 162.5011 82.1857) (end 161.361 81.0456) (width 0.25) (layer F.Cu) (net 6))
 (segment (start 170.18 78.7726) (end 170.18 77.47) (width 0.25) (layer B.Cu) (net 6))
 (segment (start 171.437 80.0296) (end 170.18 78.7726) (width 0.25) (layer B.Cu) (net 6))
 (segment (start 162.5011 82.5236) (end 162.5011 82.1857) (width 0.25) (layer F.Cu) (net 6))
 (segment (start 162.5011 82.5236) (end 162.5011 82.4397) (width 0.25) (layer F.Cu) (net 6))
 (segment (start 170.18 77.9416) (end 170.18 77.47) (width 0.25) (layer F.Cu) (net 6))
 (segment (start 174.696 74.9496) (end 174.696 75.494) (width 0.25) (layer F.Cu) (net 7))
 (segment (start 150.312 72.9176) (end 173.299 72.9176) (width 0.25) (layer F.Cu) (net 7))
 (segment (start 173.299 72.9176) (end 174.696 74.3146) (width 0.25) (layer F.Cu) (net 7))
 (segment (start 174.696 74.3146) (end 174.696 74.9496) (width 0.25) (layer F.Cu) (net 7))
 (segment (start 148.706 74.5236) (end 150.312 72.9176) (width 0.25) (layer F.Cu) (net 7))
 (segment (start 174.696 75.494) (end 172.72 77.47) (width 0.25) (layer F.Cu) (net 7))
 (segment (start 148.5011 74.5236) (end 148.706 74.5236) (width 0.25) (layer F.Cu) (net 7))
 (segment (start 148.5011 74.5236) (end 149.6 75.6225) (width 0.25) (layer F.Cu) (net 7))
 (segment (start 149.6 75.6225) (end 149.6 79.5986) (width 0.25) (layer F.Cu) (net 7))
 (segment (start 149.6 79.5986) (end 148.675 80.5236) (width 0.25) (layer F.Cu) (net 7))
 (segment (start 148.675 80.5236) (end 148.5011 80.5236) (width 0.25) (layer F.Cu) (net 7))
 (segment (start 144.5 74.4) (end 148.3775 74.4) (width 0.25) (layer F.Cu) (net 7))
 (segment (start 148.3775 74.4) (end 148.5011 74.5236) (width 0.25) (layer F.Cu) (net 7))
 (segment (start 148.5011 78.5236) (end 146.992 78.5236) (width 0.25) (layer F.Cu) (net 9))
 (segment (start 146.992 78.5236) (end 144.724 80.7916) (width 0.25) (layer F.Cu) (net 9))
 (segment (start 144.724 80.7916) (end 144.724 82.8666) (width 0.25) (layer F.Cu) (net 9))
 (segment (start 148.5011 78.5236) (end 147.0236 78.5236) (width 0.25) (layer F.Cu) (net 9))
 (segment (start 162.5011 86.5236) (end 166.034 86.5236) (width 0.25) (layer F.Cu) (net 13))
 (segment (start 166.034 86.5236) (end 166.06 86.5496) (width 0.25) (layer F.Cu) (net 13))
 (segment (start 141.549 74.1036) (end 143.327 74.1036) (width 0.25) (layer F.Cu) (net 8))
 (segment (start 143.327 74.1036) (end 144.343 75.1196) (width 0.25) (layer F.Cu) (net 8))
 (segment (start 144.343 75.1196) (end 145.656 75.1196) (width 0.25) (layer F.Cu) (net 8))
 (segment (start 145.656 75.1196) (end 147.06 76.5236) (width 0.25) (layer F.Cu) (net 8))
 (segment (start 147.06 76.5236) (end 148.5011 76.5236) (width 0.25) (layer F.Cu) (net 8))
 (segment (start 148.5011 76.5236) (end 146.8236 76.5236) (width 0.25) (layer F.Cu) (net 8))
 (segment (start 128.325 83.575) (end 128.325 82.175) (width 0.25) (layer F.Cu) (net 17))
 (segment (start 128.325 82.175) (end 128.25 82.1) (width 0.25) (layer F.Cu) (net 17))
 (segment (start 130.525 83.575) (end 131.99 83.575) (width 0.25) (layer F.Cu) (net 18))
 (segment (start 131.99 83.575) (end 132.79 82.775) (width 0.25) (layer F.Cu) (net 18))
 (segment (start 128.65 79.8) (end 128.25 80.2) (width 0.25) (layer F.Cu) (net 18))
 (segment (start 131.6 79.8) (end 128.65 79.8) (width 0.25) (layer F.Cu) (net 18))
 (segment (start 131.6 81.585) (end 132.79 82.775) (width 0.25) (layer F.Cu) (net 18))
 (segment (start 131.6 79.8) (end 131.6 81.585) (width 0.25) (layer F.Cu) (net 18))
 (segment (start 128.325 86.675) (end 127.9 87.1) (width 0.25) (layer F.Cu) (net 19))
 (segment (start 128.325 85.475) (end 128.325 86.675) (width 0.25) (layer F.Cu) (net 19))
 (segment (start 128.75 87.1) (end 128.325 86.675) (width 0.25) (layer F.Cu) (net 19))
 (segment (start 129.5 87.1) (end 128.75 87.1) (width 0.25) (layer F.Cu) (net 19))
 (segment (start 131.1 87.1) (end 131.1 86.05) (width 0.25) (layer F.Cu) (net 20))
 (segment (start 131.1 86.05) (end 130.525 85.475) (width 0.25) (layer F.Cu) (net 20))
 (segment (start 171.437 81.6806) (end 168.092 81.6806) (width 0.25) (layer F.Cu) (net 16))
 (segment (start 164.935 78.5236) (end 162.5011 78.5236) (width 0.25) (layer F.Cu) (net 16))
 (segment (start 168.092 81.6806) (end 164.935 78.5236) (width 0.25) (layer F.Cu) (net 16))
 (segment (start 173.639 86.2476) (end 173.639 85.0686) (width 0.25) (layer F.Cu) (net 16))
 (segment (start 172.41 82.6536) (end 171.437 81.6806) (width 0.25) (layer F.Cu) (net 16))
 (segment (start 172.41 83.8396) (end 172.41 82.6536) (width 0.25) (layer F.Cu) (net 16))
 (segment (start 173.639 85.0686) (end 172.41 83.8396) (width 0.25) (layer F.Cu) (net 16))
 (segment (start 163.919 78.5236) (end 162.5011 78.5236) (width 0.25) (layer F.Cu) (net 16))
 (segment (start 171.437 83.3316) (end 168.219 83.3316) (width 0.25) (layer F.Cu) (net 15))
 (segment (start 165.411 80.5236) (end 162.5011 80.5236) (width 0.25) (layer F.Cu) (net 15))
 (segment (start 168.219 83.3316) (end 165.411 80.5236) (width 0.25) (layer F.Cu) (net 15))
 (segment (start 172.989 86.2476) (end 172.989 85.4346) (width 0.25) (layer F.Cu) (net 15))
 (segment (start 171.437 83.8826) (end 171.437 83.3316) (width 0.25) (layer F.Cu) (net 15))
 (segment (start 172.989 85.4346) (end 171.437 83.8826) (width 0.25) (layer F.Cu) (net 15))
 (segment (start 163.647 80.5376) (end 163.633 80.5236) (width 0.25) (layer F.Cu) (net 15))
 (segment (start 163.633 80.5236) (end 162.5011 80.5236) (width 0.25) (layer F.Cu) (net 15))
 (via (at 140.152 73.1716) (size 0.6) (drill 0.4) (layers F.Cu B.Cu) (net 1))
 (via (at 173.807 89.9356) (size 0.6) (drill 0.4) (layers F.Cu B.Cu) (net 2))
 (via (at 172.283 89.9356) (size 0.6) (drill 0.4) (layers F.Cu B.Cu) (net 2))
 (via (at 141.93 78.7596) (size 0.6) (drill 0.4) (layers F.Cu B.Cu) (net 2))
 (via (at 139.898 78.7596) (size 0.6) (drill 0.4) (layers F.Cu B.Cu) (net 2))
 (via (at 144.75 87.55) (size 0.6) (drill 0.4) (layers F.Cu B.Cu) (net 2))
 (via (at 161.6 88.9236) (size 0.6) (drill 0.4) (layers F.Cu B.Cu) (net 2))
 (via (at 161.6 88.2236) (size 0.6) (drill 0.4) (layers F.Cu B.Cu) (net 2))
 (via (at 136.5 80.9236) (size 0.6) (drill 0.4) (layers F.Cu B.Cu) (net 2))
 (via (at 136.5 80.1236) (size 0.6) (drill 0.4) (layers F.Cu B.Cu) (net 2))
 (via (at 128.325 84.525) (size 0.6) (drill 0.4) (layers F.Cu B.Cu) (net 2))
 (via (at 140.914 78.7596) (size 0.6) (drill 0.4) (layers F.Cu B.Cu) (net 2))
 (via (at 140.914 80.83986) (size 0.6) (drill 0.4) (layers F.Cu B.Cu) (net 2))
 (via (at 171.437 80.0296) (size 0.6) (drill 0.4) (layers F.Cu B.Cu) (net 6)))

